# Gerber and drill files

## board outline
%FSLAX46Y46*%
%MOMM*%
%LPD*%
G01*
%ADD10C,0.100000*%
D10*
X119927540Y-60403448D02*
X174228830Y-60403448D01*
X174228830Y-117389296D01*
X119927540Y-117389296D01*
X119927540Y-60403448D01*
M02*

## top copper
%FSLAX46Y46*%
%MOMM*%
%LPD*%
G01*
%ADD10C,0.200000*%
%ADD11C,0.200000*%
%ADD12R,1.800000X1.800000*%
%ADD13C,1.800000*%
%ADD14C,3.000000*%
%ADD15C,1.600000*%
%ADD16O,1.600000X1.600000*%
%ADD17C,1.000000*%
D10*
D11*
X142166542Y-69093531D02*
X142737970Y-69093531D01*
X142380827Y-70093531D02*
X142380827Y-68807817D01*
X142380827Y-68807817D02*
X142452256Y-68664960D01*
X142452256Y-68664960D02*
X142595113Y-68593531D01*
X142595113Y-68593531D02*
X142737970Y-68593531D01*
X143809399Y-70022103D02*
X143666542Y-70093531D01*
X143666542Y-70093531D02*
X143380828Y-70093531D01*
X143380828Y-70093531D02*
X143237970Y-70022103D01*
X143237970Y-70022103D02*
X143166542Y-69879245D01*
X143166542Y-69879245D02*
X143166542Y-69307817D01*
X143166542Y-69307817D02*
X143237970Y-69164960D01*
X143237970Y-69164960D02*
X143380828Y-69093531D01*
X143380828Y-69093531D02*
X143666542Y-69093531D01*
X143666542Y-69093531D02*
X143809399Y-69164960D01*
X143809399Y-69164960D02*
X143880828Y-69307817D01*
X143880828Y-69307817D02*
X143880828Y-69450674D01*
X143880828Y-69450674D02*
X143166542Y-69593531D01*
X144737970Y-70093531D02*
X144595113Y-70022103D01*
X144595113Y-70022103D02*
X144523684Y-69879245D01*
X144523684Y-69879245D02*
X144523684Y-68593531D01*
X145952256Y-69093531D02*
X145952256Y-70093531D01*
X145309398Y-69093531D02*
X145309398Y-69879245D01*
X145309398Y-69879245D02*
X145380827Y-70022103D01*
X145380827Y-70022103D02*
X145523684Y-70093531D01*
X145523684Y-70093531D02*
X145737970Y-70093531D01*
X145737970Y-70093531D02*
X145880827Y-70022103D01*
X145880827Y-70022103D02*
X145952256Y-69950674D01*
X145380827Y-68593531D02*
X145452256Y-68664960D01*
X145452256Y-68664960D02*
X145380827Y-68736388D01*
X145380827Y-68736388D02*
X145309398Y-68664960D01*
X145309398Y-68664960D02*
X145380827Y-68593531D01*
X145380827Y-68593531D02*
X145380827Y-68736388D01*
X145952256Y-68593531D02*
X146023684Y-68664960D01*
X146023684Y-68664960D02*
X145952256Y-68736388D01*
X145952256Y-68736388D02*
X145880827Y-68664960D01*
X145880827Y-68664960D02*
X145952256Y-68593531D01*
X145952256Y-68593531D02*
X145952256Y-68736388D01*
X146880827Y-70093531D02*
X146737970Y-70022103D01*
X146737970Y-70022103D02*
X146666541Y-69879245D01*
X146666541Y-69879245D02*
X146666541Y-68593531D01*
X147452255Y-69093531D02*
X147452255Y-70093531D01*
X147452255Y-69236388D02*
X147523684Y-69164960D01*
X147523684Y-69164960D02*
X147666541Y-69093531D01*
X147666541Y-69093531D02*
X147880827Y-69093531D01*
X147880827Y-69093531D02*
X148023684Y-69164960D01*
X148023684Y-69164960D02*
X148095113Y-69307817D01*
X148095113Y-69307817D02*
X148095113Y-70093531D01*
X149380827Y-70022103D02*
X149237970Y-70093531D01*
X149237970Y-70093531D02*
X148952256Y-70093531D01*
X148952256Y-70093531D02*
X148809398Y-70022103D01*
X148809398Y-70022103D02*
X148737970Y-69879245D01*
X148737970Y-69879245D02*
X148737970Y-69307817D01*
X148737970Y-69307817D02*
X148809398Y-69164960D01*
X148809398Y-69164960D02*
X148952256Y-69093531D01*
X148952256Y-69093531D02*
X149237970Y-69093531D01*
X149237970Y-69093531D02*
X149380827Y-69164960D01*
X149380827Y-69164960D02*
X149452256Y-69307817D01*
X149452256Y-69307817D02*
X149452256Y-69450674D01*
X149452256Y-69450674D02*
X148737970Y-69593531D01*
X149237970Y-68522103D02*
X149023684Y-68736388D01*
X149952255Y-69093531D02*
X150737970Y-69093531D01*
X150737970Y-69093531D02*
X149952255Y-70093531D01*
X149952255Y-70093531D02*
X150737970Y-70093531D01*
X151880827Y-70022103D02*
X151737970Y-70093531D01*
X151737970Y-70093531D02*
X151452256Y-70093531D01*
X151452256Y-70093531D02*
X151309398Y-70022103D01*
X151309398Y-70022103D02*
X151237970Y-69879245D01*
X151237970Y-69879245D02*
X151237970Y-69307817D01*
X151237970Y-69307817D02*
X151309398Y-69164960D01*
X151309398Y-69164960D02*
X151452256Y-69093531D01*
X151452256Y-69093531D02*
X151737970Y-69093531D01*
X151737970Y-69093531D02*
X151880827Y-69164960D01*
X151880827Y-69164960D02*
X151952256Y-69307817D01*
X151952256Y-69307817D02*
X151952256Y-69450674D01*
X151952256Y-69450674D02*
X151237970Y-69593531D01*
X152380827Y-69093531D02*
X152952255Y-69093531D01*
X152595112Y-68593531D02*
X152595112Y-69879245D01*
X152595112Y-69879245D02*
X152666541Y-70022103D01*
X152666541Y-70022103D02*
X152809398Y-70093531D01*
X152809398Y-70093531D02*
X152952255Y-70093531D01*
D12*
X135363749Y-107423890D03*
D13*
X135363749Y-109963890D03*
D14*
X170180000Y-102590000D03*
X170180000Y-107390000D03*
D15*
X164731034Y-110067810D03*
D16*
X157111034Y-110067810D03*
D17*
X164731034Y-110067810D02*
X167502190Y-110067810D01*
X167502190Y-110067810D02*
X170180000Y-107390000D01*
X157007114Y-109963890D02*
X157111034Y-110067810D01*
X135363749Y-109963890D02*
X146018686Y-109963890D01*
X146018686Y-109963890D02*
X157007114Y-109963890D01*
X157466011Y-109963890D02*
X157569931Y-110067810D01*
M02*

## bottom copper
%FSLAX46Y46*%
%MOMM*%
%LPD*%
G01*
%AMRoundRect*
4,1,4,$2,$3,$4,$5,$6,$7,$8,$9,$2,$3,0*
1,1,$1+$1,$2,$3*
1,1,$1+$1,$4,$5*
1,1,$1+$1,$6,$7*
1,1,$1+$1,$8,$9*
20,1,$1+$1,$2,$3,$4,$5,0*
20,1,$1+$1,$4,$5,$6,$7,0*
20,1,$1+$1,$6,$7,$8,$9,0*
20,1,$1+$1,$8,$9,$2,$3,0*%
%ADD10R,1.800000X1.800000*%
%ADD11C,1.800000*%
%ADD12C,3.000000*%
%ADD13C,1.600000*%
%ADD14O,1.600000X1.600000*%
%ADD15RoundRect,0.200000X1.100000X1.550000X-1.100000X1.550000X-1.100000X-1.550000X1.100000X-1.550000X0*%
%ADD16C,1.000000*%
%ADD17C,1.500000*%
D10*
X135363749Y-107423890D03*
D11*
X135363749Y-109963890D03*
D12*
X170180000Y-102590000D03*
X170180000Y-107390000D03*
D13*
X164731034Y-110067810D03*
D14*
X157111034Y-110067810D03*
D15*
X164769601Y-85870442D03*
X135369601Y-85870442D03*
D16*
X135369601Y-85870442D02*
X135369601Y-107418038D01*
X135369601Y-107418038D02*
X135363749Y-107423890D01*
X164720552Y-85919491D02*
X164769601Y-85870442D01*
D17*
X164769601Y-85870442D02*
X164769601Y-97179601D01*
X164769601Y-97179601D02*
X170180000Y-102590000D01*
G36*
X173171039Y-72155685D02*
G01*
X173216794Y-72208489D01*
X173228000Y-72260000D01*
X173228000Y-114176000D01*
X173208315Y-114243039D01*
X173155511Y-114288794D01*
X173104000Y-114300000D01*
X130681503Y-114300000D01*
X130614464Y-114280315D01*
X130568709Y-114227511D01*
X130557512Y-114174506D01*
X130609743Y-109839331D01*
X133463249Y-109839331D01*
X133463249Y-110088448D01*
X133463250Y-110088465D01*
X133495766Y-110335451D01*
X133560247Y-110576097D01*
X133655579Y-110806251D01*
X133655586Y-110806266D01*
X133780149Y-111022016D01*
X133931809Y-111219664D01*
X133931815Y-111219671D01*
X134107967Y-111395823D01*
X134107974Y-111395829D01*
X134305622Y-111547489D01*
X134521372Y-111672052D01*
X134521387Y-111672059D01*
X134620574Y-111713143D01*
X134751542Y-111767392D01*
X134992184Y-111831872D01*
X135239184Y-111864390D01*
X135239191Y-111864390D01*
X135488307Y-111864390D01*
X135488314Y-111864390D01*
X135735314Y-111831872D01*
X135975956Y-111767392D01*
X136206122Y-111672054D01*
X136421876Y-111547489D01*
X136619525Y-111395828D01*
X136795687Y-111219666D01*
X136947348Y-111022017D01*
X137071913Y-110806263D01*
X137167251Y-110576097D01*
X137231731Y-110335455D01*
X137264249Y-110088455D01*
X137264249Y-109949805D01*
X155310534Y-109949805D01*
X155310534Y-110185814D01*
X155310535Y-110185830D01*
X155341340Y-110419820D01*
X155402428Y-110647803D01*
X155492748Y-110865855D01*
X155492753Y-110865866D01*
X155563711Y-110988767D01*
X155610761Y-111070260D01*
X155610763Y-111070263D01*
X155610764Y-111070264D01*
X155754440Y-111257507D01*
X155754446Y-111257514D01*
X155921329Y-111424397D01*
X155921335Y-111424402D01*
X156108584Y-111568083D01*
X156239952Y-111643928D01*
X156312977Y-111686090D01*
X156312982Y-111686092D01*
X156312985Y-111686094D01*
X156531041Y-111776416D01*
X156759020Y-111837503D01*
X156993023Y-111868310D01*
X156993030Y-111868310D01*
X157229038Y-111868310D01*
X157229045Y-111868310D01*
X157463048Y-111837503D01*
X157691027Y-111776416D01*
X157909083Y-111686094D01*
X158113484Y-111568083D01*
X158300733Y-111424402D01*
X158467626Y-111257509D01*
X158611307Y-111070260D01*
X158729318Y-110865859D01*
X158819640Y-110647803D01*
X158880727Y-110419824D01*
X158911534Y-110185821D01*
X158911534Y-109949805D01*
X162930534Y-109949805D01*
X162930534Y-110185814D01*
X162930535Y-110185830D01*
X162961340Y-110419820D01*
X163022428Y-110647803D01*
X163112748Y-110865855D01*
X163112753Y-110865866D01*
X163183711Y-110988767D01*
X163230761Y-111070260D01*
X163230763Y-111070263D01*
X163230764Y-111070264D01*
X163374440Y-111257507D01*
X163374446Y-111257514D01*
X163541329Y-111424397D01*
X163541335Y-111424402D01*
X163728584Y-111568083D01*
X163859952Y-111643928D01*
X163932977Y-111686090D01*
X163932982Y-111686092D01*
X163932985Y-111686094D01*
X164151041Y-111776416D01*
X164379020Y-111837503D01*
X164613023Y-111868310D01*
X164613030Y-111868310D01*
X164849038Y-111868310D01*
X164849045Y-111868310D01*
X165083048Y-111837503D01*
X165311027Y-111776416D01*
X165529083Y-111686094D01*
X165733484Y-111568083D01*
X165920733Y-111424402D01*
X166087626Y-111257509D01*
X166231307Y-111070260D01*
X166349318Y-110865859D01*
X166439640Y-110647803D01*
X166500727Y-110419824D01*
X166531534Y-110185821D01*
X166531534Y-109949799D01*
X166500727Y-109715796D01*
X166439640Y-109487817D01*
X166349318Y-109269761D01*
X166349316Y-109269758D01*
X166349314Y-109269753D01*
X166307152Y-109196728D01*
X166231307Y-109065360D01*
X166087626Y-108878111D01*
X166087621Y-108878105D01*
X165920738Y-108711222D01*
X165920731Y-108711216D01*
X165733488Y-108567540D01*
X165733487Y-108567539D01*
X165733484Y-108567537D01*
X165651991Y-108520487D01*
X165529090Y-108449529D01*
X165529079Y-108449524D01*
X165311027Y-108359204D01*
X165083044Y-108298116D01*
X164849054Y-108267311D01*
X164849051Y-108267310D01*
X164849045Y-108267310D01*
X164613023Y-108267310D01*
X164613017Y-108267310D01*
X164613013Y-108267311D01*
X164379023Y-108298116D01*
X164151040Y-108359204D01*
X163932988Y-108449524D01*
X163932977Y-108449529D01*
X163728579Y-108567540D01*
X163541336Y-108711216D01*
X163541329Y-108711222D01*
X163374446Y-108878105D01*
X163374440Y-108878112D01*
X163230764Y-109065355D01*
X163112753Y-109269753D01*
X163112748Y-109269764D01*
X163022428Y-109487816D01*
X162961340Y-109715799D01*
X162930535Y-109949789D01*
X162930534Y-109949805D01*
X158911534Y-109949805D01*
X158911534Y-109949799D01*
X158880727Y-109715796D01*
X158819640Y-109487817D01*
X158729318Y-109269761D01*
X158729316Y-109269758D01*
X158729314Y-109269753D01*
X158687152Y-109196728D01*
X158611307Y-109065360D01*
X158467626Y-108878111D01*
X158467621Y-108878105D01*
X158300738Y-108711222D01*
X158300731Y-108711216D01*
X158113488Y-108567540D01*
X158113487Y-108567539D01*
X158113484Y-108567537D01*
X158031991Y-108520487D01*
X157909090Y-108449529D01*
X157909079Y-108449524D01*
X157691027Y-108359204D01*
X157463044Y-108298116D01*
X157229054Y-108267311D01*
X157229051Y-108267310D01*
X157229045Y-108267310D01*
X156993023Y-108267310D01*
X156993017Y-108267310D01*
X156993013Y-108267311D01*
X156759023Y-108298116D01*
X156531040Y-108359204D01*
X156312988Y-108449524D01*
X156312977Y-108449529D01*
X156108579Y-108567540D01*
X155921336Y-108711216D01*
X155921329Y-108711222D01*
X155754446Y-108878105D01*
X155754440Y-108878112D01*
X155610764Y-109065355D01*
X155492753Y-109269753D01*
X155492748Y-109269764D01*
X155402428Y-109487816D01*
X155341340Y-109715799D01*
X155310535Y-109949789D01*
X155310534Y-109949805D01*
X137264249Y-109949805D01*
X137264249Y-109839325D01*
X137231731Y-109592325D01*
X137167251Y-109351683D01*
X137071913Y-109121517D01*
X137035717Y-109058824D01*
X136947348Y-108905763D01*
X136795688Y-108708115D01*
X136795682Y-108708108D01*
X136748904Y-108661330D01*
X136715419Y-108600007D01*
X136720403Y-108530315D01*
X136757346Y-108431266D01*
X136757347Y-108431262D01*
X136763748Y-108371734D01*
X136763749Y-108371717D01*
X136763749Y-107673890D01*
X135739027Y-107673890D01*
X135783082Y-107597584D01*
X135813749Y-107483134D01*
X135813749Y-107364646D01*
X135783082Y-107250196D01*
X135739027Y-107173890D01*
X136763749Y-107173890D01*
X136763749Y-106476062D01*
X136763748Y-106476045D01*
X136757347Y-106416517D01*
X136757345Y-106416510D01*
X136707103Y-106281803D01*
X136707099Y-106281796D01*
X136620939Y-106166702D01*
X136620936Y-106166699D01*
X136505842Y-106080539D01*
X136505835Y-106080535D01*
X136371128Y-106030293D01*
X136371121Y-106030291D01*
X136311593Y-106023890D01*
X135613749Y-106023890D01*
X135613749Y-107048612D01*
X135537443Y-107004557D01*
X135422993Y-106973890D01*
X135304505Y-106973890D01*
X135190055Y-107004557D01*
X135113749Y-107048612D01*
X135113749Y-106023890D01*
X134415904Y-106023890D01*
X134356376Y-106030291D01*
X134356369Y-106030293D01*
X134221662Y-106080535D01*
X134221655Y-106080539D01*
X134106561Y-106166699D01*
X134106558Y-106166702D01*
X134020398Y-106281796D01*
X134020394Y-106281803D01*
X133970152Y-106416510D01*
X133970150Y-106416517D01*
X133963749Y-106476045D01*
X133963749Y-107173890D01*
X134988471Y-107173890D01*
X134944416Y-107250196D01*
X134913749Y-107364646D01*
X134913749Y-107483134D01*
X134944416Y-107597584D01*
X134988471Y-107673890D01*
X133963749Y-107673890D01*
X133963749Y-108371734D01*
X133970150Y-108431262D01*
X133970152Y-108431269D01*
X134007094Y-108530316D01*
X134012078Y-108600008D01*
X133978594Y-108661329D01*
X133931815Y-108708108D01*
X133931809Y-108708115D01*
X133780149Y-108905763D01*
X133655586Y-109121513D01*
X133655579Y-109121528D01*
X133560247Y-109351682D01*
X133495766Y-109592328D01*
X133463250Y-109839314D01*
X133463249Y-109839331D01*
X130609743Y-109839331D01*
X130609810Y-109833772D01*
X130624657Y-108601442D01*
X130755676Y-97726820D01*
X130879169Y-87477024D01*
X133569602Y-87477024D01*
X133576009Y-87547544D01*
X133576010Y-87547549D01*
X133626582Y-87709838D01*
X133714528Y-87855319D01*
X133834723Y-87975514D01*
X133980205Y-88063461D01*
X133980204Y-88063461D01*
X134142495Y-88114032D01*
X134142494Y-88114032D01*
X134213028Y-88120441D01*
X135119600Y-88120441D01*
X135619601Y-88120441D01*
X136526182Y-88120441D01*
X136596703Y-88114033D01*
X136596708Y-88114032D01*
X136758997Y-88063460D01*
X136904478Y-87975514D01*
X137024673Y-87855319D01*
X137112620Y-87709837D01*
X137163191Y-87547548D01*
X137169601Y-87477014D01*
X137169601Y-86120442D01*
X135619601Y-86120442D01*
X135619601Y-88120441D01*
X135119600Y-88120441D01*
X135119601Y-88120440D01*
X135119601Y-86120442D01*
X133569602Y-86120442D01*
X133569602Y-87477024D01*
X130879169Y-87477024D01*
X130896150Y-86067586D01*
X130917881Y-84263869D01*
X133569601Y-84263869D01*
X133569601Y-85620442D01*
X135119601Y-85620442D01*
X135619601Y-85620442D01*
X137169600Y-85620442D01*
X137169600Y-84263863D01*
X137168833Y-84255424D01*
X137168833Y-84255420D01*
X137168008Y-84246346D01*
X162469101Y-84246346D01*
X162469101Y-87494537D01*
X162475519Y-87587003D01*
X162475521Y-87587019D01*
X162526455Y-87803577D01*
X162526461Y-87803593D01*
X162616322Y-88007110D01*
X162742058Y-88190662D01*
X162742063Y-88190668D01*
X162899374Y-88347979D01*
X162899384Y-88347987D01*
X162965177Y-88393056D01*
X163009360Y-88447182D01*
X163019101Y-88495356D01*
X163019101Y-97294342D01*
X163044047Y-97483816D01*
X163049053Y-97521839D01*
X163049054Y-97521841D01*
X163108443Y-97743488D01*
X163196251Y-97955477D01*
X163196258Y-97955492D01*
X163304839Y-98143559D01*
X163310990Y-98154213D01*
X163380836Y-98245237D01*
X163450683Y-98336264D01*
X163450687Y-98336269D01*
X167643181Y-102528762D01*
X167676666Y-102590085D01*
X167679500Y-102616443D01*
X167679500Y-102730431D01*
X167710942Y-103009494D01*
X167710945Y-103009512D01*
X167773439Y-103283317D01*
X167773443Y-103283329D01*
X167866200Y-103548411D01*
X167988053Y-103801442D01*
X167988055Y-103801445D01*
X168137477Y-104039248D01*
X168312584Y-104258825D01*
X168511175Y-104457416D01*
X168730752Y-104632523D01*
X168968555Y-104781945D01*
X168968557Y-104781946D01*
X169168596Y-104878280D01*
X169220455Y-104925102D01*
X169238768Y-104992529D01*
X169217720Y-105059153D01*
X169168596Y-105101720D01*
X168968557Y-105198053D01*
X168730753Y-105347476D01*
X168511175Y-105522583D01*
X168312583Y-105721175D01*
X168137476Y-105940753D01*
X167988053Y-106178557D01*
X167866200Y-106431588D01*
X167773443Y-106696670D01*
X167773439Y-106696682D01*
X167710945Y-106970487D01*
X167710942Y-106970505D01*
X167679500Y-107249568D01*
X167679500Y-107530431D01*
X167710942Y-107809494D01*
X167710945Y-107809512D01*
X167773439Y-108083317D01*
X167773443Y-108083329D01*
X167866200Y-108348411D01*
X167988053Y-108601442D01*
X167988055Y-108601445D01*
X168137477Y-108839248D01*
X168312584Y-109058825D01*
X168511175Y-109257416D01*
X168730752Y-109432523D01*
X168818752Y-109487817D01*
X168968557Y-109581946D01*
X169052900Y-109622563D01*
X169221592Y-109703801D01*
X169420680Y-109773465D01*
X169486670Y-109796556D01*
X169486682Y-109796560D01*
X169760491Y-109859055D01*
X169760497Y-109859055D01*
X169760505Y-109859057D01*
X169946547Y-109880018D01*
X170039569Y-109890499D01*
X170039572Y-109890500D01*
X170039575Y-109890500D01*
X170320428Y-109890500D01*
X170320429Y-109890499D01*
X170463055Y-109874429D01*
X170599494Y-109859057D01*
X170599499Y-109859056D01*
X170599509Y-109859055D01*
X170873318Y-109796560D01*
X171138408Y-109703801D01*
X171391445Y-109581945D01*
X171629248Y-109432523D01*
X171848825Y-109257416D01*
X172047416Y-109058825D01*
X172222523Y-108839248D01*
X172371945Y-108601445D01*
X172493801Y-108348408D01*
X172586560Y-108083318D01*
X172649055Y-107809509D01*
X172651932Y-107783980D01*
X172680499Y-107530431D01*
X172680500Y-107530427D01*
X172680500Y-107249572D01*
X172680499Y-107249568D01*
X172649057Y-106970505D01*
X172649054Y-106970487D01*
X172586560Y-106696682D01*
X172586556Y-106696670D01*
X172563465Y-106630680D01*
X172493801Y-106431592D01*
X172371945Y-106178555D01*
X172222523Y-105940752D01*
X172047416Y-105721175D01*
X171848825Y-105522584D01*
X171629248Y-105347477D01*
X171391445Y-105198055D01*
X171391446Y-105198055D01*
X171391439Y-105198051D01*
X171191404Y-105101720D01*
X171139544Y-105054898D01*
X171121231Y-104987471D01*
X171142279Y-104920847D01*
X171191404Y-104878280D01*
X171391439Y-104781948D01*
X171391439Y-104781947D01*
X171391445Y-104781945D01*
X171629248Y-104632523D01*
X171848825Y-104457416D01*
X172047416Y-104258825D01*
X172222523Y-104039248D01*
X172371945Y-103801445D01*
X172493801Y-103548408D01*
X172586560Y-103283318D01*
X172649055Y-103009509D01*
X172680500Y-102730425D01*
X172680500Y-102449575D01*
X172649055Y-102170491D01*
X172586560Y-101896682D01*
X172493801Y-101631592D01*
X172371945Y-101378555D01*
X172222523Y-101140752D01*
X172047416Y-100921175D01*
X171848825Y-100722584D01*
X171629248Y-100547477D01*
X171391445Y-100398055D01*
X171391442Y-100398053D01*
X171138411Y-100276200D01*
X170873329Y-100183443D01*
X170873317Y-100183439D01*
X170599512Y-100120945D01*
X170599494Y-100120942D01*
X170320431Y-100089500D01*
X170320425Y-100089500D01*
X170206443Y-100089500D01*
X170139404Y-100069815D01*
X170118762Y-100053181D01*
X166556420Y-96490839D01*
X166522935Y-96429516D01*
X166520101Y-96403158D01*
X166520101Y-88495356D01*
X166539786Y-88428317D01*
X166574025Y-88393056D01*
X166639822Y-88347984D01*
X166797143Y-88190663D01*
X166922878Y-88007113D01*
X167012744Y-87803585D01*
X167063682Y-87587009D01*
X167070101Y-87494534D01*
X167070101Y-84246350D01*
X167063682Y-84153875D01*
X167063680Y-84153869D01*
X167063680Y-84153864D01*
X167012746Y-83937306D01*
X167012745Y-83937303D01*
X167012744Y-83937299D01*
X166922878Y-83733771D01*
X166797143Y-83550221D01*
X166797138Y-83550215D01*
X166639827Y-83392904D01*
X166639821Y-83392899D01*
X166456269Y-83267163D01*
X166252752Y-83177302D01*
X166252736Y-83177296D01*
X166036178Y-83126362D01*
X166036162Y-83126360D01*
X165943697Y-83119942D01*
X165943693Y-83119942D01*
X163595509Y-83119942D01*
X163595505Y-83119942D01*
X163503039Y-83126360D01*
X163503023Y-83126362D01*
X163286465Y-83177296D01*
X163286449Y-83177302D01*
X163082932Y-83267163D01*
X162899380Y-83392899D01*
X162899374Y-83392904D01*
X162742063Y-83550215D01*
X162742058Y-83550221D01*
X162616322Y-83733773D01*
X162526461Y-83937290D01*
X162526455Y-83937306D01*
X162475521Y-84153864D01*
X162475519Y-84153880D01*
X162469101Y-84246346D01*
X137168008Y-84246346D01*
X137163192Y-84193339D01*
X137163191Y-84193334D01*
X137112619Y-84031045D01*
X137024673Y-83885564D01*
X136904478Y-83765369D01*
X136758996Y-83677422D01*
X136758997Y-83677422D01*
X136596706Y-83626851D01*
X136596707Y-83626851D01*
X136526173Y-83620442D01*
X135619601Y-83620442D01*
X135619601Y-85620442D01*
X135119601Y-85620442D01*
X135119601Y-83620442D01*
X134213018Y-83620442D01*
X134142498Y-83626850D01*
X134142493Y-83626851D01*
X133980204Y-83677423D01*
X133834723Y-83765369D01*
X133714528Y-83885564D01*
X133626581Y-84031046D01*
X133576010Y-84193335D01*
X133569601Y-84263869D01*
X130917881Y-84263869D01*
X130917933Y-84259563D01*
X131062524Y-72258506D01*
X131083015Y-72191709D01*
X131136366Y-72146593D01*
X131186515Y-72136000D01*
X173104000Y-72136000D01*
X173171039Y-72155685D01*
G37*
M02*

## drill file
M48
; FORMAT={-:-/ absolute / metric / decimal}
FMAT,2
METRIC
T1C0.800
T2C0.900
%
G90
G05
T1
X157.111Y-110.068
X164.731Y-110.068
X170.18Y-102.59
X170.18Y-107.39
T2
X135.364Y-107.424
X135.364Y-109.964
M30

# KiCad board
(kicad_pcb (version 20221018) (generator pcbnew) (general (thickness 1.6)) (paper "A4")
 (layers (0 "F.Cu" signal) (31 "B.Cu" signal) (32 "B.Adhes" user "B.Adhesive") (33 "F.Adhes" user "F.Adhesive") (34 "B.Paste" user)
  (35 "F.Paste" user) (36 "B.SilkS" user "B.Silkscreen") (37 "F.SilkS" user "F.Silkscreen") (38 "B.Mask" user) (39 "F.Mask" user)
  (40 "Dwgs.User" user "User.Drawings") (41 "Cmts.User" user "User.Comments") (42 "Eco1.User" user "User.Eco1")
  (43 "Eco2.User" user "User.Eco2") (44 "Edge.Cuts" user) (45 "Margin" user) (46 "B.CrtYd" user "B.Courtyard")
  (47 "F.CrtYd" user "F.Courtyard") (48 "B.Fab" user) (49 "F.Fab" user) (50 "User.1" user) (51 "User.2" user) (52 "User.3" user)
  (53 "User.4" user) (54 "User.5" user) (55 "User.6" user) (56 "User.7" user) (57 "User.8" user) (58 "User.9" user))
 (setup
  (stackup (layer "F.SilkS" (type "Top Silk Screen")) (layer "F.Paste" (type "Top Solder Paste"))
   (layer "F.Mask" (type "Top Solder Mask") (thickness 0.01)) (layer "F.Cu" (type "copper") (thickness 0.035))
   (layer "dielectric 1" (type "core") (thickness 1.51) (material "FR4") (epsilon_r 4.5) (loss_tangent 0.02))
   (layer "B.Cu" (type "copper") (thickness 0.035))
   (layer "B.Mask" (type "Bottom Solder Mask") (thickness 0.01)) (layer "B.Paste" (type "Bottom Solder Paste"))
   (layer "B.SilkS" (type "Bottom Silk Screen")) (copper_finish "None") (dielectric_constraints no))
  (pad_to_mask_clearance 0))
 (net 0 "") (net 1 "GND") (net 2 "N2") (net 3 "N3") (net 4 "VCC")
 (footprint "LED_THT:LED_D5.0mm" (layer "F.Cu") (at 135.363749 107.42389 -90)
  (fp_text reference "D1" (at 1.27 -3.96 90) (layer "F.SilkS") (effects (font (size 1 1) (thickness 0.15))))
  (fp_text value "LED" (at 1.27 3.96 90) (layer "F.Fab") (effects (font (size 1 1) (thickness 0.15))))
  (pad "1" thru_hole rect (at 0 0 270) (size 1.8 1.8) (drill 0.9) (layers "*.Cu" "*.Mask") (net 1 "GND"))
  (pad "2" thru_hole circle (at 2.54 0 270) (size 1.8 1.8) (drill 0.9) (layers "*.Cu" "*.Mask") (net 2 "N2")))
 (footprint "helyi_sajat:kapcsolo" (layer "F.Cu") (at 170.18 97.79)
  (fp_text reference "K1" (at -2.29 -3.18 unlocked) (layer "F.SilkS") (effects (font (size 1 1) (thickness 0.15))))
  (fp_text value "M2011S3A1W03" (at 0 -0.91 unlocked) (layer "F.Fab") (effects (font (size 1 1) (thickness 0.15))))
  (pad "2" thru_hole circle (at 0 4.8) (size 3 3) (drill 0.8) (layers "*.Cu" "*.Mask") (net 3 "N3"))
  (pad "3" thru_hole circle (at 0 9.6) (size 3 3) (drill 0.8) (layers "*.Cu" "*.Mask") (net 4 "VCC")))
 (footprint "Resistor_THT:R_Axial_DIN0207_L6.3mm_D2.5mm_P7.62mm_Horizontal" (layer "F.Cu") (at 164.731034 110.06781 180)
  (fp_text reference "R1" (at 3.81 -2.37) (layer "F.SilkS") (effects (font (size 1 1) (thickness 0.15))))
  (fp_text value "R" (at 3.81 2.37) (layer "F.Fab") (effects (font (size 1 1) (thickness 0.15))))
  (pad "1" thru_hole circle (at 0 0 180) (size 1.6 1.6) (drill 0.8) (layers "*.Cu" "*.Mask") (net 4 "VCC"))
  (pad "2" thru_hole oval (at 7.62 0 180) (size 1.6 1.6) (drill 0.8) (layers "*.Cu" "*.Mask") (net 2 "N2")))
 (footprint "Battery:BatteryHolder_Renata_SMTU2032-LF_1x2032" (layer "B.Cu") (at 150.069601 85.870442 180)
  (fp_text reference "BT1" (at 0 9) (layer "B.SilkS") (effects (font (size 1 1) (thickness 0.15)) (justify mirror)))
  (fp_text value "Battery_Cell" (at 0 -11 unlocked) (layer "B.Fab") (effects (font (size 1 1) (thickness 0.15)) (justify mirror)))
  (pad "1" smd roundrect (at -14.7 0 180) (size 2.6 3.5) (layers "B.Cu" "B.Paste" "B.Mask") (roundrect_rratio 0.07692307692) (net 3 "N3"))
  (pad "2" smd roundrect (at 14.7 0 180) (size 2.6 3.5) (layers "B.Cu" "B.Paste" "B.Mask") (roundrect_rratio 0.07692307692) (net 1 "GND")))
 (gr_rect (start 119.92754 60.403448) (end 174.22883 117.389296) (stroke (width 0.1) (type default)) (fill none) (layer "Edge.Cuts"))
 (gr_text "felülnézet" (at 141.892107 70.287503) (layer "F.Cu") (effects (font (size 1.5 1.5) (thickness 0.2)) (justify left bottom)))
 (segment (start 164.731034 110.06781) (end 167.50219 110.06781) (width 1) (layer "F.Cu") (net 4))
 (segment (start 167.50219 110.06781) (end 170.18 107.39) (width 1) (layer "F.Cu") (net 4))
 (segment (start 135.369601 85.870442) (end 135.369601 107.418038) (width 1) (layer "B.Cu") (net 1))
 (segment (start 135.369601 107.418038) (end 135.363749 107.42389) (width 1) (layer "B.Cu") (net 1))
 (segment (start 157.007114 109.96389) (end 157.111034 110.06781) (width 1) (layer "F.Cu") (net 2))
 (segment (start 135.363749 109.96389) (end 146.018686 109.96389) (width 1) (layer "F.Cu") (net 2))
 (segment (start 146.018686 109.96389) (end 157.007114 109.96389) (width 1) (layer "F.Cu") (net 2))
 (segment (start 157.466011 109.96389) (end 157.569931 110.06781) (width 1) (layer "F.Cu") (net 2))
 (segment (start 164.720552 85.919491) (end 164.769601 85.870442) (width 1) (layer "B.Cu") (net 3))
 (segment (start 164.769601 85.870442) (end 164.769601 97.179601) (width 1.5) (layer "B.Cu") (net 3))
 (segment (start 164.769601 97.179601) (end 170.18 102.59) (width 1.5) (layer "B.Cu") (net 3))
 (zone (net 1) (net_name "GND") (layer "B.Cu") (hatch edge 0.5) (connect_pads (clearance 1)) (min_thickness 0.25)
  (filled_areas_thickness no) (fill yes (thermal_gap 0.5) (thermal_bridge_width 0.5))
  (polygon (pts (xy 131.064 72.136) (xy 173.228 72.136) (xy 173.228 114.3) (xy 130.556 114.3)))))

